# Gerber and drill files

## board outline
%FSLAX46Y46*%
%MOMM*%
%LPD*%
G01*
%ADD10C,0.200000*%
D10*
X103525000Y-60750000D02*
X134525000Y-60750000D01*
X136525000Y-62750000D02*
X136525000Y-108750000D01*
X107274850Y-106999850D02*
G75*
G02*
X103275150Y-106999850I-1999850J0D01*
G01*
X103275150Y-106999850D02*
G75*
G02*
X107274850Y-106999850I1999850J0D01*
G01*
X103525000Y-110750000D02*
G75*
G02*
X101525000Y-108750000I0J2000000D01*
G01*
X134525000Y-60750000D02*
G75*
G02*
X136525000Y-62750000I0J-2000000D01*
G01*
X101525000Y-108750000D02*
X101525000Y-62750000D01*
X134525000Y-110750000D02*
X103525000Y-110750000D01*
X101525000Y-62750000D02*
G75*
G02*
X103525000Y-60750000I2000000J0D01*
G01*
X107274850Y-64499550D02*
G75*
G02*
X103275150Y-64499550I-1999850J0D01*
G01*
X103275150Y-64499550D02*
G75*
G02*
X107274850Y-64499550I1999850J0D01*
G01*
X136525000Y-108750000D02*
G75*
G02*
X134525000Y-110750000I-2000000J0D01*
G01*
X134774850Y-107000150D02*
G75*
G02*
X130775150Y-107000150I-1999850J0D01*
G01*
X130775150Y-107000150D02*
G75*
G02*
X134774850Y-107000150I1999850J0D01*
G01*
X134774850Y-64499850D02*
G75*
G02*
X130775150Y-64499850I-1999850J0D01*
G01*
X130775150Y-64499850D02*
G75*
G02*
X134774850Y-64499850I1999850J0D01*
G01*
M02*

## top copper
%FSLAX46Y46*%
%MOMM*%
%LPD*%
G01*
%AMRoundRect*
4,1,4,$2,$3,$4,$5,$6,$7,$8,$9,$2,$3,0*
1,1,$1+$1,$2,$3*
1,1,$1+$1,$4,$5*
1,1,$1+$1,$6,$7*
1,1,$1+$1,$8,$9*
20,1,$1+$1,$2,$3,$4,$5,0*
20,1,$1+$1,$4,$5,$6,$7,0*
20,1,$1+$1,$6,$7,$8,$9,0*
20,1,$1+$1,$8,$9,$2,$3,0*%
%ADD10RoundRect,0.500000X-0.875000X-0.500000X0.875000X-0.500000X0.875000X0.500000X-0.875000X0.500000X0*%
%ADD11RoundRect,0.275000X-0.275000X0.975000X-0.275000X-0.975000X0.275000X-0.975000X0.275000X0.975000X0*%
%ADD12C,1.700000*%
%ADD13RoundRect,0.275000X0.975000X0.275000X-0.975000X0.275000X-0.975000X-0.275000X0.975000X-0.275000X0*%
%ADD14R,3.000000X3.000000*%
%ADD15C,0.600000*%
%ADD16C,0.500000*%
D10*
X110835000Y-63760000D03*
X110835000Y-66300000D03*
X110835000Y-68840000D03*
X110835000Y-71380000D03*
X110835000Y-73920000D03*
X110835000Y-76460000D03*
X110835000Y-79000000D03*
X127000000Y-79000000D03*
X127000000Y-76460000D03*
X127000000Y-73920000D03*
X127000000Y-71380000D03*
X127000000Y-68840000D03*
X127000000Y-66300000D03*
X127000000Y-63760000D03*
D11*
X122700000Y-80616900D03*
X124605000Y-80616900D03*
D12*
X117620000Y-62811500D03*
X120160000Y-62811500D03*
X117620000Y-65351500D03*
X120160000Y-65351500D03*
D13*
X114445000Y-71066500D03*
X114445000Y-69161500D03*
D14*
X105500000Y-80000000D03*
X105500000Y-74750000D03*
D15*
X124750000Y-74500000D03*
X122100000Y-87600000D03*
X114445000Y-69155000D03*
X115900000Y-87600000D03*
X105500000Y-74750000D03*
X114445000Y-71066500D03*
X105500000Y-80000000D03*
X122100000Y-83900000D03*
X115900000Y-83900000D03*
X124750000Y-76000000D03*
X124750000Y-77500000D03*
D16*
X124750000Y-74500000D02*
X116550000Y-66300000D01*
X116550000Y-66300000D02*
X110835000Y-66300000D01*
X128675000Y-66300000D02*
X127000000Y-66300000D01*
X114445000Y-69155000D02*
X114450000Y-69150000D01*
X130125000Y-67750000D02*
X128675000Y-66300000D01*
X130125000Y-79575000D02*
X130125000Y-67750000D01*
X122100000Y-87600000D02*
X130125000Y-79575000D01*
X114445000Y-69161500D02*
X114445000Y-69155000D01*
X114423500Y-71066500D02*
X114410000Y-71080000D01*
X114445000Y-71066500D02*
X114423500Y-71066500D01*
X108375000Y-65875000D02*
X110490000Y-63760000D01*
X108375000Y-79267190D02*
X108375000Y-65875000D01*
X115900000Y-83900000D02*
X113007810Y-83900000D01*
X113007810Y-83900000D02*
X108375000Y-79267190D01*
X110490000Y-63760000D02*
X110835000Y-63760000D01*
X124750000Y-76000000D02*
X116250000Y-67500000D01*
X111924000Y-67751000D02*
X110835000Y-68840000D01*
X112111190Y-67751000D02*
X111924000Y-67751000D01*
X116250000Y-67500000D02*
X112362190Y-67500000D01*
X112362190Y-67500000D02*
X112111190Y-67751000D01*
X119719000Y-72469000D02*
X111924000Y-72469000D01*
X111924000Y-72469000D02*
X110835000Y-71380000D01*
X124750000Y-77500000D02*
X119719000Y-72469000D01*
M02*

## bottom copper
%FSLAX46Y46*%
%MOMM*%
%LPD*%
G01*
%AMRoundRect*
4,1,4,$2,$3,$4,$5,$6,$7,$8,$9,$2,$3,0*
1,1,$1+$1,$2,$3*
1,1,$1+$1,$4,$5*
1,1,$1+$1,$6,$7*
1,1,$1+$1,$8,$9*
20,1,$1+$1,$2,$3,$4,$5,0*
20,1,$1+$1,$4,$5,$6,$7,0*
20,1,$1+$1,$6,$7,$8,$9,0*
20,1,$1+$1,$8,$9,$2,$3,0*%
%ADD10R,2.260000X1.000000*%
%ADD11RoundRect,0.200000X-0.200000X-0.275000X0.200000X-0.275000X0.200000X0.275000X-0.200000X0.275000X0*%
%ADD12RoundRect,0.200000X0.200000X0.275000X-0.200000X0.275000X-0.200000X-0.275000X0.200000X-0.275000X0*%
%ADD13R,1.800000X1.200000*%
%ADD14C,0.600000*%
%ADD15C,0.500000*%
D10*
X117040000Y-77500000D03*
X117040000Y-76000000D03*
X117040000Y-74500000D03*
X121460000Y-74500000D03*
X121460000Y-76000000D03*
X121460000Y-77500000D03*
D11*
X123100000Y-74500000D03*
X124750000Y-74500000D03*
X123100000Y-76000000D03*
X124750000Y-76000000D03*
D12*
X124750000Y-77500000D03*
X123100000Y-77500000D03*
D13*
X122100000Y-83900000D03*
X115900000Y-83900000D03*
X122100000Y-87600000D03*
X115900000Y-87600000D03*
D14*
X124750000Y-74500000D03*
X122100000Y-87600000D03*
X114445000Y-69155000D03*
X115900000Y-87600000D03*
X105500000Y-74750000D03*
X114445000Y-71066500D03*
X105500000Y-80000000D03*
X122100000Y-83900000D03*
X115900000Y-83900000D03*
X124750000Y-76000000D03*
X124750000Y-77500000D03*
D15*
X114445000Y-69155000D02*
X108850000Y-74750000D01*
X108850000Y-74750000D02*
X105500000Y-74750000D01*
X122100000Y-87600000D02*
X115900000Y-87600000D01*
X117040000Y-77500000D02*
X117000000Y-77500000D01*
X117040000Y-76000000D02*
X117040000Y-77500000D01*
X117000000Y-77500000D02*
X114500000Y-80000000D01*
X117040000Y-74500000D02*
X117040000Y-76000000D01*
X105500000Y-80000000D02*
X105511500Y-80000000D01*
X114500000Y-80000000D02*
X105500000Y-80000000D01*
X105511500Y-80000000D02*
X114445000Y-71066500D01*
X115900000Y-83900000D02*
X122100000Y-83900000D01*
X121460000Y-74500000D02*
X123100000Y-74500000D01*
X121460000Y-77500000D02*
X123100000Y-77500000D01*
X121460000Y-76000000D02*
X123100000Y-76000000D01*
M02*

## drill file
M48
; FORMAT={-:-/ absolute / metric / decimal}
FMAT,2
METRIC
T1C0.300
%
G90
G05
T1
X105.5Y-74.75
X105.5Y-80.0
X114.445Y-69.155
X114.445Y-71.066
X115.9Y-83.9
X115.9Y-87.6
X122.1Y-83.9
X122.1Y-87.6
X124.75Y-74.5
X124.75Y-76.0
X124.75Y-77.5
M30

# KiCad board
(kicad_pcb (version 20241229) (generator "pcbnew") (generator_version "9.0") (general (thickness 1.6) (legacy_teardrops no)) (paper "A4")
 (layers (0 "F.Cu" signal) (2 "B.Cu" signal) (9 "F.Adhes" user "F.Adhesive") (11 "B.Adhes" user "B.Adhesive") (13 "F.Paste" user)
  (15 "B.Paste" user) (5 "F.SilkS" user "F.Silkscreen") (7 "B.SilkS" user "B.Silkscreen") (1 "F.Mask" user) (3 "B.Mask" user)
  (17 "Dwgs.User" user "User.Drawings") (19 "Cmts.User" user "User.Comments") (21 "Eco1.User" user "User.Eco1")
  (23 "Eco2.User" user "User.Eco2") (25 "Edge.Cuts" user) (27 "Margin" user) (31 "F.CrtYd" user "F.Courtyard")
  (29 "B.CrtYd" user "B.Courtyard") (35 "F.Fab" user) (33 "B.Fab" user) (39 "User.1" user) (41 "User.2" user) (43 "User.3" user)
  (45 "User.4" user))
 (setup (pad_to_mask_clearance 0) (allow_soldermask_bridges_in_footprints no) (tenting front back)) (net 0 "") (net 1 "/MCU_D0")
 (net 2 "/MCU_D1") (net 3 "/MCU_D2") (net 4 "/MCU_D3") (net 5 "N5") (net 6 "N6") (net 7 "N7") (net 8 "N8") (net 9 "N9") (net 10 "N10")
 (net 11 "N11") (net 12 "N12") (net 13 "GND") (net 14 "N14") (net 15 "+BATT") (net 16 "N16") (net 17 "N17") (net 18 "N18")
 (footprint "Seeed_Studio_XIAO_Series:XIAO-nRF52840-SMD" (layer "F.Cu") (at 110 81.88)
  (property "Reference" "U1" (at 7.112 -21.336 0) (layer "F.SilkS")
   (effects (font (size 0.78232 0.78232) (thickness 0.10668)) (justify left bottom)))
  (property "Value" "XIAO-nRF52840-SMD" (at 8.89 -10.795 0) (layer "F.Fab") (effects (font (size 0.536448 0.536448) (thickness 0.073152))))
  (pad "1" smd roundrect (at 0.835 -18.12) (size 2.75 2) (layers "F.Cu" "F.Mask" "F.Paste") (roundrect_rratio 0.25) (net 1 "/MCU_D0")
   (solder_mask_margin 0.0508) (thermal_bridge_angle 45))
  (pad "2" smd roundrect (at 0.835 -15.58) (size 2.75 2) (layers "F.Cu" "F.Mask" "F.Paste") (roundrect_rratio 0.25) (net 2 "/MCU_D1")
   (solder_mask_margin 0.0508) (thermal_bridge_angle 45))
  (pad "3" smd roundrect (at 0.835 -13.04) (size 2.75 2) (layers "F.Cu" "F.Mask" "F.Paste") (roundrect_rratio 0.25) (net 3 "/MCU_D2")
   (solder_mask_margin 0.0508) (thermal_bridge_angle 45))
  (pad "4" smd roundrect (at 0.835 -10.5) (size 2.75 2) (layers "F.Cu" "F.Mask" "F.Paste") (roundrect_rratio 0.25) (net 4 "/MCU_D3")
   (solder_mask_margin 0.0508) (thermal_bridge_angle 45))
  (pad "5" smd roundrect (at 0.835 -7.96) (size 2.75 2) (layers "F.Cu" "F.Mask" "F.Paste") (roundrect_rratio 0.25) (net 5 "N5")
   (solder_mask_margin 0.0508) (thermal_bridge_angle 45))
  (pad "6" smd roundrect (at 0.835 -5.42) (size 2.75 2) (layers "F.Cu" "F.Mask" "F.Paste") (roundrect_rratio 0.25) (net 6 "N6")
   (solder_mask_margin 0.0508) (thermal_bridge_angle 45))
  (pad "7" smd roundrect (at 0.835 -2.88) (size 2.75 2) (layers "F.Cu" "F.Mask" "F.Paste") (roundrect_rratio 0.25) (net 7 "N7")
   (solder_mask_margin 0.0508) (thermal_bridge_angle 45))
  (pad "8" smd roundrect (at 17 -2.88) (size 2.75 2) (layers "F.Cu" "F.Mask" "F.Paste") (roundrect_rratio 0.25) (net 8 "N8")
   (solder_mask_margin 0.0508) (thermal_bridge_angle 45))
  (pad "9" smd roundrect (at 17 -5.42) (size 2.75 2) (layers "F.Cu" "F.Mask" "F.Paste") (roundrect_rratio 0.25) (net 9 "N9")
   (solder_mask_margin 0.0508) (thermal_bridge_angle 45))
  (pad "10" smd roundrect (at 17 -7.96) (size 2.75 2) (layers "F.Cu" "F.Mask" "F.Paste") (roundrect_rratio 0.25) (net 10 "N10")
   (solder_mask_margin 0.0508) (thermal_bridge_angle 45))
  (pad "11" smd roundrect (at 17 -10.5) (size 2.75 2) (layers "F.Cu" "F.Mask" "F.Paste") (roundrect_rratio 0.25) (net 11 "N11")
   (solder_mask_margin 0.0508) (thermal_bridge_angle 45))
  (pad "12" smd roundrect (at 17 -13.04) (size 2.75 2) (layers "F.Cu" "F.Mask" "F.Paste") (roundrect_rratio 0.25) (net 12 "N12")
   (solder_mask_margin 0.0508) (thermal_bridge_angle 45))
  (pad "13" smd roundrect (at 17 -15.58) (size 2.75 2) (layers "F.Cu" "F.Mask" "F.Paste") (roundrect_rratio 0.25) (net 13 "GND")
   (solder_mask_margin 0.0508) (thermal_bridge_angle 45))
  (pad "14" smd roundrect (at 17 -18.12) (size 2.75 2) (layers "F.Cu" "F.Mask" "F.Paste") (roundrect_rratio 0.25) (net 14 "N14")
   (solder_mask_margin 0.0508) (thermal_bridge_angle 45))
  (pad "17" smd roundrect (at 12.7 -1.2631 270) (size 2.5 1.1) (layers "F.Cu" "F.Mask" "F.Paste") (roundrect_rratio 0.25)
   (solder_mask_margin 0.0508) (thermal_bridge_angle 45))
  (pad "18" smd roundrect (at 14.605 -1.2631 270) (size 2.5 1.1) (layers "F.Cu" "F.Mask" "F.Paste") (roundrect_rratio 0.25)
   (solder_mask_margin 0.0508) (thermal_bridge_angle 45))
  (pad "19" smd circle (at 7.62 -19.0685) (size 1.7 1.7) (layers "F.Cu" "F.Mask" "F.Paste"))
  (pad "20" smd circle (at 10.16 -19.0685) (size 1.7 1.7) (layers "F.Cu" "F.Mask" "F.Paste"))
  (pad "21" smd circle (at 7.62 -16.5285) (size 1.7 1.7) (layers "F.Cu" "F.Mask" "F.Paste"))
  (pad "22" smd circle (at 10.16 -16.5285) (size 1.7 1.7) (layers "F.Cu" "F.Mask" "F.Paste"))
  (pad "32" smd roundrect (at 4.445 -10.8135 180) (size 2.5 1.1) (layers "F.Cu" "F.Mask" "F.Paste") (roundrect_rratio 0.25) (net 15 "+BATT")
   (solder_mask_margin 0.0508) (thermal_bridge_angle 45))
  (pad "33" smd roundrect (at 4.445 -12.7185 180) (size 2.5 1.1) (layers "F.Cu" "F.Mask" "F.Paste") (roundrect_rratio 0.25) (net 13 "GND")
   (solder_mask_margin 0.0508) (thermal_bridge_angle 45)))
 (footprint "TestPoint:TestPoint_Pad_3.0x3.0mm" (layer "F.Cu") (at 105.5 80 90)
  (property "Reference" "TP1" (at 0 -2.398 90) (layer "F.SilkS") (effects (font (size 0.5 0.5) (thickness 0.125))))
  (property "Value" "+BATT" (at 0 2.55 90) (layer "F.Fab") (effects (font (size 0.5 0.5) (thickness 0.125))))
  (pad "1" smd rect (at 0 0 90) (size 3 3) (layers "F.Cu" "F.Mask") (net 15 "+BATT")))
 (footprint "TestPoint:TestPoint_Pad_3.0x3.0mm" (layer "F.Cu") (at 105.5 74.75 90)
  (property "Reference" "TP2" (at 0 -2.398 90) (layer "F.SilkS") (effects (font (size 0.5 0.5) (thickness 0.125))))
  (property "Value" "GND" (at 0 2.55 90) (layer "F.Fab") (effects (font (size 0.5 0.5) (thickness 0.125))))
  (pad "1" smd rect (at 0 0 90) (size 3 3) (layers "F.Cu" "F.Mask") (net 13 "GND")))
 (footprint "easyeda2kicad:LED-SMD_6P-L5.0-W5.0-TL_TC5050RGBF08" (layer "B.Cu") (at 119.25 76)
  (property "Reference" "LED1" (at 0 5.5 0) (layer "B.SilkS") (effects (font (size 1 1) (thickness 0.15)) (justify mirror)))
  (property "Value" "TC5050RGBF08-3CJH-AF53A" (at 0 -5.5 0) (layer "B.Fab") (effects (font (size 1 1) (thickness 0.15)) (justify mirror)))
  (pad "1" smd rect (at -2.21 1.5) (size 2.26 1) (layers "B.Cu" "B.Mask" "B.Paste") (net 15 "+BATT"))
  (pad "2" smd rect (at -2.21 0) (size 2.26 1) (layers "B.Cu" "B.Mask" "B.Paste") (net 15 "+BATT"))
  (pad "3" smd rect (at -2.21 -1.5) (size 2.26 1) (layers "B.Cu" "B.Mask" "B.Paste") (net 15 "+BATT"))
  (pad "4" smd rect (at 2.21 -1.5) (size 2.26 1) (layers "B.Cu" "B.Mask" "B.Paste") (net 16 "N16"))
  (pad "5" smd rect (at 2.21 0) (size 2.26 1) (layers "B.Cu" "B.Mask" "B.Paste") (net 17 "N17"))
  (pad "6" smd rect (at 2.21 1.5) (size 2.26 1) (layers "B.Cu" "B.Mask" "B.Paste") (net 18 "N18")))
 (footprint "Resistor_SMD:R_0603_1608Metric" (layer "B.Cu") (at 123.925 74.5)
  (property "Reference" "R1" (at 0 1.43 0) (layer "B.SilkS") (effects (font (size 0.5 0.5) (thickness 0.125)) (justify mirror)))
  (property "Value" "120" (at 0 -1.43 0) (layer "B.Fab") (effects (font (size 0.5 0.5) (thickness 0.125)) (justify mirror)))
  (pad "1" smd roundrect (at -0.825 0) (size 0.8 0.95) (layers "B.Cu" "B.Mask" "B.Paste") (roundrect_rratio 0.25) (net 16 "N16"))
  (pad "2" smd roundrect (at 0.825 0) (size 0.8 0.95) (layers "B.Cu" "B.Mask" "B.Paste") (roundrect_rratio 0.25) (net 2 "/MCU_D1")))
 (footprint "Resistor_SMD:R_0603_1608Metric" (layer "B.Cu") (at 123.925 76)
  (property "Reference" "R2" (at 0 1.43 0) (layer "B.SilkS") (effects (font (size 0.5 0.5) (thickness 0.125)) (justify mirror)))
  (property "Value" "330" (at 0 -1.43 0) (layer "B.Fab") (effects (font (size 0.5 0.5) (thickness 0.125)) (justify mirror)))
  (pad "1" smd roundrect (at -0.825 0) (size 0.8 0.95) (layers "B.Cu" "B.Mask" "B.Paste") (roundrect_rratio 0.25) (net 17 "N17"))
  (pad "2" smd roundrect (at 0.825 0) (size 0.8 0.95) (layers "B.Cu" "B.Mask" "B.Paste") (roundrect_rratio 0.25) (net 3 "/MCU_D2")))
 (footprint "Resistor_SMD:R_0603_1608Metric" (layer "B.Cu") (at 123.925 77.5 180)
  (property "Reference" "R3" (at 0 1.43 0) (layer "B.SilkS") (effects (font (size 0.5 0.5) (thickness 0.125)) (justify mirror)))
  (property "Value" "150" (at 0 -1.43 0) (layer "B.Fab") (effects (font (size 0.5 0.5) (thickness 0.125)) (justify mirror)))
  (pad "1" smd roundrect (at -0.825 0 180) (size 0.8 0.95) (layers "B.Cu" "B.Mask" "B.Paste") (roundrect_rratio 0.25) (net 4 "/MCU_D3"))
  (pad "2" smd roundrect (at 0.825 0 180) (size 0.8 0.95) (layers "B.Cu" "B.Mask" "B.Paste") (roundrect_rratio 0.25) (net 18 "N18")))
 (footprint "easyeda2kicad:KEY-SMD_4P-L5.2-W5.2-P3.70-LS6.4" (layer "B.Cu") (at 119 85.75 180)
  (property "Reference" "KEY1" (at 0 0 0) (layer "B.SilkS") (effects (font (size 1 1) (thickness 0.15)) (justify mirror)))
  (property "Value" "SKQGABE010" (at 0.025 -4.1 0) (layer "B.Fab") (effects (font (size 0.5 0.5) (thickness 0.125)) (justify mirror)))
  (pad "1" smd rect (at -3.1 1.85 180) (size 1.8 1.2) (layers "B.Cu" "B.Mask" "B.Paste") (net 1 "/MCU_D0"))
  (pad "2" smd rect (at 3.1 1.85 180) (size 1.8 1.2) (layers "B.Cu" "B.Mask" "B.Paste") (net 1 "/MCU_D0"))
  (pad "3" smd rect (at -3.1 -1.85 180) (size 1.8 1.2) (layers "B.Cu" "B.Mask" "B.Paste") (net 13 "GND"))
  (pad "4" smd rect (at 3.1 -1.85 180) (size 1.8 1.2) (layers "B.Cu" "B.Mask" "B.Paste") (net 13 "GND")))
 (gr_line (start 103.525 60.75) (end 134.525 60.75) (stroke (width 0.2) (type default)) (layer "Edge.Cuts"))
 (gr_line (start 136.525 62.75) (end 136.525 108.75) (stroke (width 0.2) (type default)) (layer "Edge.Cuts"))
 (gr_circle (center 105.275 106.99985) (end 106.405 108.64985) (stroke (width 0.2) (type solid)) (fill no) (layer "Edge.Cuts"))
 (gr_arc (start 103.525 110.75) (mid 102.110786 110.164214) (end 101.525 108.75) (stroke (width 0.2) (type default)) (layer "Edge.Cuts"))
 (gr_arc (start 134.525 60.75) (mid 135.939214 61.335786) (end 136.525 62.75) (stroke (width 0.2) (type default)) (layer "Edge.Cuts"))
 (gr_line (start 101.525 108.75) (end 101.525 62.75) (stroke (width 0.2) (type default)) (layer "Edge.Cuts"))
 (gr_line (start 134.525 110.75) (end 103.525 110.75) (stroke (width 0.2) (type default)) (layer "Edge.Cuts"))
 (gr_arc (start 101.525 62.75) (mid 102.110786 61.335786) (end 103.525 60.75) (stroke (width 0.2) (type default)) (layer "Edge.Cuts"))
 (gr_circle (center 105.275 64.49955) (end 106.405 66.14955) (stroke (width 0.2) (type solid)) (fill no) (layer "Edge.Cuts"))
 (gr_arc (start 136.525 108.75) (mid 135.939214 110.164214) (end 134.525 110.75) (stroke (width 0.2) (type default)) (layer "Edge.Cuts"))
 (gr_circle (center 132.775 107.00015) (end 133.905 108.65015) (stroke (width 0.2) (type solid)) (fill no) (layer "Edge.Cuts"))
 (gr_circle (center 132.775 64.49985) (end 133.905 66.14985) (stroke (width 0.2) (type solid)) (fill no) (layer "Edge.Cuts"))
 (segment (start 124.75 74.5) (end 116.55 66.3) (width 0.5) (layer "F.Cu") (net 2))
 (segment (start 116.55 66.3) (end 110.835 66.3) (width 0.5) (layer "F.Cu") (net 2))
 (via (at 124.75 74.5) (size 0.6) (drill 0.3) (layers "F.Cu" "B.Cu") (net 2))
 (segment (start 128.675 66.3) (end 127 66.3) (width 0.5) (layer "F.Cu") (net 13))
 (segment (start 114.445 69.155) (end 114.45 69.15) (width 0.5) (layer "F.Cu") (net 13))
 (segment (start 130.125 67.75) (end 128.675 66.3) (width 0.5) (layer "F.Cu") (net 13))
 (segment (start 130.125 79.575) (end 130.125 67.75) (width 0.5) (layer "F.Cu") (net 13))
 (segment (start 122.1 87.6) (end 130.125 79.575) (width 0.5) (layer "F.Cu") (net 13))
 (segment (start 114.445 69.1615) (end 114.445 69.155) (width 0.5) (layer "F.Cu") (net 13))
 (via (at 122.1 87.6) (size 0.6) (drill 0.3) (layers "F.Cu" "B.Cu") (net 13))
 (via (at 114.445 69.155) (size 0.6) (drill 0.3) (layers "F.Cu" "B.Cu") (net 13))
 (via (at 115.9 87.6) (size 0.6) (drill 0.3) (layers "F.Cu" "B.Cu") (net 13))
 (via (at 105.5 74.75) (size 0.6) (drill 0.3) (layers "F.Cu" "B.Cu") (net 13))
 (segment (start 114.445 69.155) (end 108.85 74.75) (width 0.5) (layer "B.Cu") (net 13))
 (segment (start 108.85 74.75) (end 105.5 74.75) (width 0.5) (layer "B.Cu") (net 13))
 (segment (start 122.1 87.6) (end 115.9 87.6) (width 0.5) (layer "B.Cu") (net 13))
 (segment (start 114.4235 71.0665) (end 114.41 71.08) (width 0.5) (layer "F.Cu") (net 15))
 (segment (start 114.445 71.0665) (end 114.4235 71.0665) (width 0.5) (layer "F.Cu") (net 15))
 (via (at 114.445 71.0665) (size 0.6) (drill 0.3) (layers "F.Cu" "B.Cu") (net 15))
 (via (at 105.5 80) (size 0.6) (drill 0.3) (layers "F.Cu" "B.Cu") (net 15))
 (segment (start 117.04 77.5) (end 117 77.5) (width 0.5) (layer "B.Cu") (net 15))
 (segment (start 117.04 76) (end 117.04 77.5) (width 0.5) (layer "B.Cu") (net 15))
 (segment (start 117 77.5) (end 114.5 80) (width 0.5) (layer "B.Cu") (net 15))
 (segment (start 117.04 74.5) (end 117.04 76) (width 0.5) (layer "B.Cu") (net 15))
 (segment (start 105.5 80) (end 105.5115 80) (width 0.5) (layer "B.Cu") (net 15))
 (segment (start 114.5 80) (end 105.5 80) (width 0.5) (layer "B.Cu") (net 15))
 (segment (start 105.5115 80) (end 114.445 71.0665) (width 0.5) (layer "B.Cu") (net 15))
 (segment (start 108.375 65.875) (end 110.49 63.76) (width 0.5) (layer "F.Cu") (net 1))
 (segment (start 108.375 79.26719) (end 108.375 65.875) (width 0.5) (layer "F.Cu") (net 1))
 (segment (start 115.9 83.9) (end 113.00781 83.9) (width 0.5) (layer "F.Cu") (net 1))
 (segment (start 113.00781 83.9) (end 108.375 79.26719) (width 0.5) (layer "F.Cu") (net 1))
 (segment (start 110.49 63.76) (end 110.835 63.76) (width 0.5) (layer "F.Cu") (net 1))
 (via (at 122.1 83.9) (size 0.6) (drill 0.3) (layers "F.Cu" "B.Cu") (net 1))
 (via (at 115.9 83.9) (size 0.6) (drill 0.3) (layers "F.Cu" "B.Cu") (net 1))
 (segment (start 115.9 83.9) (end 122.1 83.9) (width 0.5) (layer "B.Cu") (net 1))
 (segment (start 124.75 76) (end 116.25 67.5) (width 0.5) (layer "F.Cu") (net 3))
 (segment (start 111.924 67.751) (end 110.835 68.84) (width 0.5) (layer "F.Cu") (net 3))
 (segment (start 112.11119 67.751) (end 111.924 67.751) (width 0.5) (layer "F.Cu") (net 3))
 (segment (start 116.25 67.5) (end 112.36219 67.5) (width 0.5) (layer "F.Cu") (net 3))
 (segment (start 112.36219 67.5) (end 112.11119 67.751) (width 0.5) (layer "F.Cu") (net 3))
 (via (at 124.75 76) (size 0.6) (drill 0.3) (layers "F.Cu" "B.Cu") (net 3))
 (segment (start 119.719 72.469) (end 111.924 72.469) (width 0.5) (layer "F.Cu") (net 4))
 (segment (start 111.924 72.469) (end 110.835 71.38) (width 0.5) (layer "F.Cu") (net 4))
 (segment (start 124.75 77.5) (end 119.719 72.469) (width 0.5) (layer "F.Cu") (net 4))
 (via (at 124.75 77.5) (size 0.6) (drill 0.3) (layers "F.Cu" "B.Cu") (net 4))
 (segment (start 121.46 74.5) (end 123.1 74.5) (width 0.5) (layer "B.Cu") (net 16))
 (segment (start 121.46 77.5) (end 123.1 77.5) (width 0.5) (layer "B.Cu") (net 18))
 (segment (start 121.46 76) (end 123.1 76) (width 0.5) (layer "B.Cu") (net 17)))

